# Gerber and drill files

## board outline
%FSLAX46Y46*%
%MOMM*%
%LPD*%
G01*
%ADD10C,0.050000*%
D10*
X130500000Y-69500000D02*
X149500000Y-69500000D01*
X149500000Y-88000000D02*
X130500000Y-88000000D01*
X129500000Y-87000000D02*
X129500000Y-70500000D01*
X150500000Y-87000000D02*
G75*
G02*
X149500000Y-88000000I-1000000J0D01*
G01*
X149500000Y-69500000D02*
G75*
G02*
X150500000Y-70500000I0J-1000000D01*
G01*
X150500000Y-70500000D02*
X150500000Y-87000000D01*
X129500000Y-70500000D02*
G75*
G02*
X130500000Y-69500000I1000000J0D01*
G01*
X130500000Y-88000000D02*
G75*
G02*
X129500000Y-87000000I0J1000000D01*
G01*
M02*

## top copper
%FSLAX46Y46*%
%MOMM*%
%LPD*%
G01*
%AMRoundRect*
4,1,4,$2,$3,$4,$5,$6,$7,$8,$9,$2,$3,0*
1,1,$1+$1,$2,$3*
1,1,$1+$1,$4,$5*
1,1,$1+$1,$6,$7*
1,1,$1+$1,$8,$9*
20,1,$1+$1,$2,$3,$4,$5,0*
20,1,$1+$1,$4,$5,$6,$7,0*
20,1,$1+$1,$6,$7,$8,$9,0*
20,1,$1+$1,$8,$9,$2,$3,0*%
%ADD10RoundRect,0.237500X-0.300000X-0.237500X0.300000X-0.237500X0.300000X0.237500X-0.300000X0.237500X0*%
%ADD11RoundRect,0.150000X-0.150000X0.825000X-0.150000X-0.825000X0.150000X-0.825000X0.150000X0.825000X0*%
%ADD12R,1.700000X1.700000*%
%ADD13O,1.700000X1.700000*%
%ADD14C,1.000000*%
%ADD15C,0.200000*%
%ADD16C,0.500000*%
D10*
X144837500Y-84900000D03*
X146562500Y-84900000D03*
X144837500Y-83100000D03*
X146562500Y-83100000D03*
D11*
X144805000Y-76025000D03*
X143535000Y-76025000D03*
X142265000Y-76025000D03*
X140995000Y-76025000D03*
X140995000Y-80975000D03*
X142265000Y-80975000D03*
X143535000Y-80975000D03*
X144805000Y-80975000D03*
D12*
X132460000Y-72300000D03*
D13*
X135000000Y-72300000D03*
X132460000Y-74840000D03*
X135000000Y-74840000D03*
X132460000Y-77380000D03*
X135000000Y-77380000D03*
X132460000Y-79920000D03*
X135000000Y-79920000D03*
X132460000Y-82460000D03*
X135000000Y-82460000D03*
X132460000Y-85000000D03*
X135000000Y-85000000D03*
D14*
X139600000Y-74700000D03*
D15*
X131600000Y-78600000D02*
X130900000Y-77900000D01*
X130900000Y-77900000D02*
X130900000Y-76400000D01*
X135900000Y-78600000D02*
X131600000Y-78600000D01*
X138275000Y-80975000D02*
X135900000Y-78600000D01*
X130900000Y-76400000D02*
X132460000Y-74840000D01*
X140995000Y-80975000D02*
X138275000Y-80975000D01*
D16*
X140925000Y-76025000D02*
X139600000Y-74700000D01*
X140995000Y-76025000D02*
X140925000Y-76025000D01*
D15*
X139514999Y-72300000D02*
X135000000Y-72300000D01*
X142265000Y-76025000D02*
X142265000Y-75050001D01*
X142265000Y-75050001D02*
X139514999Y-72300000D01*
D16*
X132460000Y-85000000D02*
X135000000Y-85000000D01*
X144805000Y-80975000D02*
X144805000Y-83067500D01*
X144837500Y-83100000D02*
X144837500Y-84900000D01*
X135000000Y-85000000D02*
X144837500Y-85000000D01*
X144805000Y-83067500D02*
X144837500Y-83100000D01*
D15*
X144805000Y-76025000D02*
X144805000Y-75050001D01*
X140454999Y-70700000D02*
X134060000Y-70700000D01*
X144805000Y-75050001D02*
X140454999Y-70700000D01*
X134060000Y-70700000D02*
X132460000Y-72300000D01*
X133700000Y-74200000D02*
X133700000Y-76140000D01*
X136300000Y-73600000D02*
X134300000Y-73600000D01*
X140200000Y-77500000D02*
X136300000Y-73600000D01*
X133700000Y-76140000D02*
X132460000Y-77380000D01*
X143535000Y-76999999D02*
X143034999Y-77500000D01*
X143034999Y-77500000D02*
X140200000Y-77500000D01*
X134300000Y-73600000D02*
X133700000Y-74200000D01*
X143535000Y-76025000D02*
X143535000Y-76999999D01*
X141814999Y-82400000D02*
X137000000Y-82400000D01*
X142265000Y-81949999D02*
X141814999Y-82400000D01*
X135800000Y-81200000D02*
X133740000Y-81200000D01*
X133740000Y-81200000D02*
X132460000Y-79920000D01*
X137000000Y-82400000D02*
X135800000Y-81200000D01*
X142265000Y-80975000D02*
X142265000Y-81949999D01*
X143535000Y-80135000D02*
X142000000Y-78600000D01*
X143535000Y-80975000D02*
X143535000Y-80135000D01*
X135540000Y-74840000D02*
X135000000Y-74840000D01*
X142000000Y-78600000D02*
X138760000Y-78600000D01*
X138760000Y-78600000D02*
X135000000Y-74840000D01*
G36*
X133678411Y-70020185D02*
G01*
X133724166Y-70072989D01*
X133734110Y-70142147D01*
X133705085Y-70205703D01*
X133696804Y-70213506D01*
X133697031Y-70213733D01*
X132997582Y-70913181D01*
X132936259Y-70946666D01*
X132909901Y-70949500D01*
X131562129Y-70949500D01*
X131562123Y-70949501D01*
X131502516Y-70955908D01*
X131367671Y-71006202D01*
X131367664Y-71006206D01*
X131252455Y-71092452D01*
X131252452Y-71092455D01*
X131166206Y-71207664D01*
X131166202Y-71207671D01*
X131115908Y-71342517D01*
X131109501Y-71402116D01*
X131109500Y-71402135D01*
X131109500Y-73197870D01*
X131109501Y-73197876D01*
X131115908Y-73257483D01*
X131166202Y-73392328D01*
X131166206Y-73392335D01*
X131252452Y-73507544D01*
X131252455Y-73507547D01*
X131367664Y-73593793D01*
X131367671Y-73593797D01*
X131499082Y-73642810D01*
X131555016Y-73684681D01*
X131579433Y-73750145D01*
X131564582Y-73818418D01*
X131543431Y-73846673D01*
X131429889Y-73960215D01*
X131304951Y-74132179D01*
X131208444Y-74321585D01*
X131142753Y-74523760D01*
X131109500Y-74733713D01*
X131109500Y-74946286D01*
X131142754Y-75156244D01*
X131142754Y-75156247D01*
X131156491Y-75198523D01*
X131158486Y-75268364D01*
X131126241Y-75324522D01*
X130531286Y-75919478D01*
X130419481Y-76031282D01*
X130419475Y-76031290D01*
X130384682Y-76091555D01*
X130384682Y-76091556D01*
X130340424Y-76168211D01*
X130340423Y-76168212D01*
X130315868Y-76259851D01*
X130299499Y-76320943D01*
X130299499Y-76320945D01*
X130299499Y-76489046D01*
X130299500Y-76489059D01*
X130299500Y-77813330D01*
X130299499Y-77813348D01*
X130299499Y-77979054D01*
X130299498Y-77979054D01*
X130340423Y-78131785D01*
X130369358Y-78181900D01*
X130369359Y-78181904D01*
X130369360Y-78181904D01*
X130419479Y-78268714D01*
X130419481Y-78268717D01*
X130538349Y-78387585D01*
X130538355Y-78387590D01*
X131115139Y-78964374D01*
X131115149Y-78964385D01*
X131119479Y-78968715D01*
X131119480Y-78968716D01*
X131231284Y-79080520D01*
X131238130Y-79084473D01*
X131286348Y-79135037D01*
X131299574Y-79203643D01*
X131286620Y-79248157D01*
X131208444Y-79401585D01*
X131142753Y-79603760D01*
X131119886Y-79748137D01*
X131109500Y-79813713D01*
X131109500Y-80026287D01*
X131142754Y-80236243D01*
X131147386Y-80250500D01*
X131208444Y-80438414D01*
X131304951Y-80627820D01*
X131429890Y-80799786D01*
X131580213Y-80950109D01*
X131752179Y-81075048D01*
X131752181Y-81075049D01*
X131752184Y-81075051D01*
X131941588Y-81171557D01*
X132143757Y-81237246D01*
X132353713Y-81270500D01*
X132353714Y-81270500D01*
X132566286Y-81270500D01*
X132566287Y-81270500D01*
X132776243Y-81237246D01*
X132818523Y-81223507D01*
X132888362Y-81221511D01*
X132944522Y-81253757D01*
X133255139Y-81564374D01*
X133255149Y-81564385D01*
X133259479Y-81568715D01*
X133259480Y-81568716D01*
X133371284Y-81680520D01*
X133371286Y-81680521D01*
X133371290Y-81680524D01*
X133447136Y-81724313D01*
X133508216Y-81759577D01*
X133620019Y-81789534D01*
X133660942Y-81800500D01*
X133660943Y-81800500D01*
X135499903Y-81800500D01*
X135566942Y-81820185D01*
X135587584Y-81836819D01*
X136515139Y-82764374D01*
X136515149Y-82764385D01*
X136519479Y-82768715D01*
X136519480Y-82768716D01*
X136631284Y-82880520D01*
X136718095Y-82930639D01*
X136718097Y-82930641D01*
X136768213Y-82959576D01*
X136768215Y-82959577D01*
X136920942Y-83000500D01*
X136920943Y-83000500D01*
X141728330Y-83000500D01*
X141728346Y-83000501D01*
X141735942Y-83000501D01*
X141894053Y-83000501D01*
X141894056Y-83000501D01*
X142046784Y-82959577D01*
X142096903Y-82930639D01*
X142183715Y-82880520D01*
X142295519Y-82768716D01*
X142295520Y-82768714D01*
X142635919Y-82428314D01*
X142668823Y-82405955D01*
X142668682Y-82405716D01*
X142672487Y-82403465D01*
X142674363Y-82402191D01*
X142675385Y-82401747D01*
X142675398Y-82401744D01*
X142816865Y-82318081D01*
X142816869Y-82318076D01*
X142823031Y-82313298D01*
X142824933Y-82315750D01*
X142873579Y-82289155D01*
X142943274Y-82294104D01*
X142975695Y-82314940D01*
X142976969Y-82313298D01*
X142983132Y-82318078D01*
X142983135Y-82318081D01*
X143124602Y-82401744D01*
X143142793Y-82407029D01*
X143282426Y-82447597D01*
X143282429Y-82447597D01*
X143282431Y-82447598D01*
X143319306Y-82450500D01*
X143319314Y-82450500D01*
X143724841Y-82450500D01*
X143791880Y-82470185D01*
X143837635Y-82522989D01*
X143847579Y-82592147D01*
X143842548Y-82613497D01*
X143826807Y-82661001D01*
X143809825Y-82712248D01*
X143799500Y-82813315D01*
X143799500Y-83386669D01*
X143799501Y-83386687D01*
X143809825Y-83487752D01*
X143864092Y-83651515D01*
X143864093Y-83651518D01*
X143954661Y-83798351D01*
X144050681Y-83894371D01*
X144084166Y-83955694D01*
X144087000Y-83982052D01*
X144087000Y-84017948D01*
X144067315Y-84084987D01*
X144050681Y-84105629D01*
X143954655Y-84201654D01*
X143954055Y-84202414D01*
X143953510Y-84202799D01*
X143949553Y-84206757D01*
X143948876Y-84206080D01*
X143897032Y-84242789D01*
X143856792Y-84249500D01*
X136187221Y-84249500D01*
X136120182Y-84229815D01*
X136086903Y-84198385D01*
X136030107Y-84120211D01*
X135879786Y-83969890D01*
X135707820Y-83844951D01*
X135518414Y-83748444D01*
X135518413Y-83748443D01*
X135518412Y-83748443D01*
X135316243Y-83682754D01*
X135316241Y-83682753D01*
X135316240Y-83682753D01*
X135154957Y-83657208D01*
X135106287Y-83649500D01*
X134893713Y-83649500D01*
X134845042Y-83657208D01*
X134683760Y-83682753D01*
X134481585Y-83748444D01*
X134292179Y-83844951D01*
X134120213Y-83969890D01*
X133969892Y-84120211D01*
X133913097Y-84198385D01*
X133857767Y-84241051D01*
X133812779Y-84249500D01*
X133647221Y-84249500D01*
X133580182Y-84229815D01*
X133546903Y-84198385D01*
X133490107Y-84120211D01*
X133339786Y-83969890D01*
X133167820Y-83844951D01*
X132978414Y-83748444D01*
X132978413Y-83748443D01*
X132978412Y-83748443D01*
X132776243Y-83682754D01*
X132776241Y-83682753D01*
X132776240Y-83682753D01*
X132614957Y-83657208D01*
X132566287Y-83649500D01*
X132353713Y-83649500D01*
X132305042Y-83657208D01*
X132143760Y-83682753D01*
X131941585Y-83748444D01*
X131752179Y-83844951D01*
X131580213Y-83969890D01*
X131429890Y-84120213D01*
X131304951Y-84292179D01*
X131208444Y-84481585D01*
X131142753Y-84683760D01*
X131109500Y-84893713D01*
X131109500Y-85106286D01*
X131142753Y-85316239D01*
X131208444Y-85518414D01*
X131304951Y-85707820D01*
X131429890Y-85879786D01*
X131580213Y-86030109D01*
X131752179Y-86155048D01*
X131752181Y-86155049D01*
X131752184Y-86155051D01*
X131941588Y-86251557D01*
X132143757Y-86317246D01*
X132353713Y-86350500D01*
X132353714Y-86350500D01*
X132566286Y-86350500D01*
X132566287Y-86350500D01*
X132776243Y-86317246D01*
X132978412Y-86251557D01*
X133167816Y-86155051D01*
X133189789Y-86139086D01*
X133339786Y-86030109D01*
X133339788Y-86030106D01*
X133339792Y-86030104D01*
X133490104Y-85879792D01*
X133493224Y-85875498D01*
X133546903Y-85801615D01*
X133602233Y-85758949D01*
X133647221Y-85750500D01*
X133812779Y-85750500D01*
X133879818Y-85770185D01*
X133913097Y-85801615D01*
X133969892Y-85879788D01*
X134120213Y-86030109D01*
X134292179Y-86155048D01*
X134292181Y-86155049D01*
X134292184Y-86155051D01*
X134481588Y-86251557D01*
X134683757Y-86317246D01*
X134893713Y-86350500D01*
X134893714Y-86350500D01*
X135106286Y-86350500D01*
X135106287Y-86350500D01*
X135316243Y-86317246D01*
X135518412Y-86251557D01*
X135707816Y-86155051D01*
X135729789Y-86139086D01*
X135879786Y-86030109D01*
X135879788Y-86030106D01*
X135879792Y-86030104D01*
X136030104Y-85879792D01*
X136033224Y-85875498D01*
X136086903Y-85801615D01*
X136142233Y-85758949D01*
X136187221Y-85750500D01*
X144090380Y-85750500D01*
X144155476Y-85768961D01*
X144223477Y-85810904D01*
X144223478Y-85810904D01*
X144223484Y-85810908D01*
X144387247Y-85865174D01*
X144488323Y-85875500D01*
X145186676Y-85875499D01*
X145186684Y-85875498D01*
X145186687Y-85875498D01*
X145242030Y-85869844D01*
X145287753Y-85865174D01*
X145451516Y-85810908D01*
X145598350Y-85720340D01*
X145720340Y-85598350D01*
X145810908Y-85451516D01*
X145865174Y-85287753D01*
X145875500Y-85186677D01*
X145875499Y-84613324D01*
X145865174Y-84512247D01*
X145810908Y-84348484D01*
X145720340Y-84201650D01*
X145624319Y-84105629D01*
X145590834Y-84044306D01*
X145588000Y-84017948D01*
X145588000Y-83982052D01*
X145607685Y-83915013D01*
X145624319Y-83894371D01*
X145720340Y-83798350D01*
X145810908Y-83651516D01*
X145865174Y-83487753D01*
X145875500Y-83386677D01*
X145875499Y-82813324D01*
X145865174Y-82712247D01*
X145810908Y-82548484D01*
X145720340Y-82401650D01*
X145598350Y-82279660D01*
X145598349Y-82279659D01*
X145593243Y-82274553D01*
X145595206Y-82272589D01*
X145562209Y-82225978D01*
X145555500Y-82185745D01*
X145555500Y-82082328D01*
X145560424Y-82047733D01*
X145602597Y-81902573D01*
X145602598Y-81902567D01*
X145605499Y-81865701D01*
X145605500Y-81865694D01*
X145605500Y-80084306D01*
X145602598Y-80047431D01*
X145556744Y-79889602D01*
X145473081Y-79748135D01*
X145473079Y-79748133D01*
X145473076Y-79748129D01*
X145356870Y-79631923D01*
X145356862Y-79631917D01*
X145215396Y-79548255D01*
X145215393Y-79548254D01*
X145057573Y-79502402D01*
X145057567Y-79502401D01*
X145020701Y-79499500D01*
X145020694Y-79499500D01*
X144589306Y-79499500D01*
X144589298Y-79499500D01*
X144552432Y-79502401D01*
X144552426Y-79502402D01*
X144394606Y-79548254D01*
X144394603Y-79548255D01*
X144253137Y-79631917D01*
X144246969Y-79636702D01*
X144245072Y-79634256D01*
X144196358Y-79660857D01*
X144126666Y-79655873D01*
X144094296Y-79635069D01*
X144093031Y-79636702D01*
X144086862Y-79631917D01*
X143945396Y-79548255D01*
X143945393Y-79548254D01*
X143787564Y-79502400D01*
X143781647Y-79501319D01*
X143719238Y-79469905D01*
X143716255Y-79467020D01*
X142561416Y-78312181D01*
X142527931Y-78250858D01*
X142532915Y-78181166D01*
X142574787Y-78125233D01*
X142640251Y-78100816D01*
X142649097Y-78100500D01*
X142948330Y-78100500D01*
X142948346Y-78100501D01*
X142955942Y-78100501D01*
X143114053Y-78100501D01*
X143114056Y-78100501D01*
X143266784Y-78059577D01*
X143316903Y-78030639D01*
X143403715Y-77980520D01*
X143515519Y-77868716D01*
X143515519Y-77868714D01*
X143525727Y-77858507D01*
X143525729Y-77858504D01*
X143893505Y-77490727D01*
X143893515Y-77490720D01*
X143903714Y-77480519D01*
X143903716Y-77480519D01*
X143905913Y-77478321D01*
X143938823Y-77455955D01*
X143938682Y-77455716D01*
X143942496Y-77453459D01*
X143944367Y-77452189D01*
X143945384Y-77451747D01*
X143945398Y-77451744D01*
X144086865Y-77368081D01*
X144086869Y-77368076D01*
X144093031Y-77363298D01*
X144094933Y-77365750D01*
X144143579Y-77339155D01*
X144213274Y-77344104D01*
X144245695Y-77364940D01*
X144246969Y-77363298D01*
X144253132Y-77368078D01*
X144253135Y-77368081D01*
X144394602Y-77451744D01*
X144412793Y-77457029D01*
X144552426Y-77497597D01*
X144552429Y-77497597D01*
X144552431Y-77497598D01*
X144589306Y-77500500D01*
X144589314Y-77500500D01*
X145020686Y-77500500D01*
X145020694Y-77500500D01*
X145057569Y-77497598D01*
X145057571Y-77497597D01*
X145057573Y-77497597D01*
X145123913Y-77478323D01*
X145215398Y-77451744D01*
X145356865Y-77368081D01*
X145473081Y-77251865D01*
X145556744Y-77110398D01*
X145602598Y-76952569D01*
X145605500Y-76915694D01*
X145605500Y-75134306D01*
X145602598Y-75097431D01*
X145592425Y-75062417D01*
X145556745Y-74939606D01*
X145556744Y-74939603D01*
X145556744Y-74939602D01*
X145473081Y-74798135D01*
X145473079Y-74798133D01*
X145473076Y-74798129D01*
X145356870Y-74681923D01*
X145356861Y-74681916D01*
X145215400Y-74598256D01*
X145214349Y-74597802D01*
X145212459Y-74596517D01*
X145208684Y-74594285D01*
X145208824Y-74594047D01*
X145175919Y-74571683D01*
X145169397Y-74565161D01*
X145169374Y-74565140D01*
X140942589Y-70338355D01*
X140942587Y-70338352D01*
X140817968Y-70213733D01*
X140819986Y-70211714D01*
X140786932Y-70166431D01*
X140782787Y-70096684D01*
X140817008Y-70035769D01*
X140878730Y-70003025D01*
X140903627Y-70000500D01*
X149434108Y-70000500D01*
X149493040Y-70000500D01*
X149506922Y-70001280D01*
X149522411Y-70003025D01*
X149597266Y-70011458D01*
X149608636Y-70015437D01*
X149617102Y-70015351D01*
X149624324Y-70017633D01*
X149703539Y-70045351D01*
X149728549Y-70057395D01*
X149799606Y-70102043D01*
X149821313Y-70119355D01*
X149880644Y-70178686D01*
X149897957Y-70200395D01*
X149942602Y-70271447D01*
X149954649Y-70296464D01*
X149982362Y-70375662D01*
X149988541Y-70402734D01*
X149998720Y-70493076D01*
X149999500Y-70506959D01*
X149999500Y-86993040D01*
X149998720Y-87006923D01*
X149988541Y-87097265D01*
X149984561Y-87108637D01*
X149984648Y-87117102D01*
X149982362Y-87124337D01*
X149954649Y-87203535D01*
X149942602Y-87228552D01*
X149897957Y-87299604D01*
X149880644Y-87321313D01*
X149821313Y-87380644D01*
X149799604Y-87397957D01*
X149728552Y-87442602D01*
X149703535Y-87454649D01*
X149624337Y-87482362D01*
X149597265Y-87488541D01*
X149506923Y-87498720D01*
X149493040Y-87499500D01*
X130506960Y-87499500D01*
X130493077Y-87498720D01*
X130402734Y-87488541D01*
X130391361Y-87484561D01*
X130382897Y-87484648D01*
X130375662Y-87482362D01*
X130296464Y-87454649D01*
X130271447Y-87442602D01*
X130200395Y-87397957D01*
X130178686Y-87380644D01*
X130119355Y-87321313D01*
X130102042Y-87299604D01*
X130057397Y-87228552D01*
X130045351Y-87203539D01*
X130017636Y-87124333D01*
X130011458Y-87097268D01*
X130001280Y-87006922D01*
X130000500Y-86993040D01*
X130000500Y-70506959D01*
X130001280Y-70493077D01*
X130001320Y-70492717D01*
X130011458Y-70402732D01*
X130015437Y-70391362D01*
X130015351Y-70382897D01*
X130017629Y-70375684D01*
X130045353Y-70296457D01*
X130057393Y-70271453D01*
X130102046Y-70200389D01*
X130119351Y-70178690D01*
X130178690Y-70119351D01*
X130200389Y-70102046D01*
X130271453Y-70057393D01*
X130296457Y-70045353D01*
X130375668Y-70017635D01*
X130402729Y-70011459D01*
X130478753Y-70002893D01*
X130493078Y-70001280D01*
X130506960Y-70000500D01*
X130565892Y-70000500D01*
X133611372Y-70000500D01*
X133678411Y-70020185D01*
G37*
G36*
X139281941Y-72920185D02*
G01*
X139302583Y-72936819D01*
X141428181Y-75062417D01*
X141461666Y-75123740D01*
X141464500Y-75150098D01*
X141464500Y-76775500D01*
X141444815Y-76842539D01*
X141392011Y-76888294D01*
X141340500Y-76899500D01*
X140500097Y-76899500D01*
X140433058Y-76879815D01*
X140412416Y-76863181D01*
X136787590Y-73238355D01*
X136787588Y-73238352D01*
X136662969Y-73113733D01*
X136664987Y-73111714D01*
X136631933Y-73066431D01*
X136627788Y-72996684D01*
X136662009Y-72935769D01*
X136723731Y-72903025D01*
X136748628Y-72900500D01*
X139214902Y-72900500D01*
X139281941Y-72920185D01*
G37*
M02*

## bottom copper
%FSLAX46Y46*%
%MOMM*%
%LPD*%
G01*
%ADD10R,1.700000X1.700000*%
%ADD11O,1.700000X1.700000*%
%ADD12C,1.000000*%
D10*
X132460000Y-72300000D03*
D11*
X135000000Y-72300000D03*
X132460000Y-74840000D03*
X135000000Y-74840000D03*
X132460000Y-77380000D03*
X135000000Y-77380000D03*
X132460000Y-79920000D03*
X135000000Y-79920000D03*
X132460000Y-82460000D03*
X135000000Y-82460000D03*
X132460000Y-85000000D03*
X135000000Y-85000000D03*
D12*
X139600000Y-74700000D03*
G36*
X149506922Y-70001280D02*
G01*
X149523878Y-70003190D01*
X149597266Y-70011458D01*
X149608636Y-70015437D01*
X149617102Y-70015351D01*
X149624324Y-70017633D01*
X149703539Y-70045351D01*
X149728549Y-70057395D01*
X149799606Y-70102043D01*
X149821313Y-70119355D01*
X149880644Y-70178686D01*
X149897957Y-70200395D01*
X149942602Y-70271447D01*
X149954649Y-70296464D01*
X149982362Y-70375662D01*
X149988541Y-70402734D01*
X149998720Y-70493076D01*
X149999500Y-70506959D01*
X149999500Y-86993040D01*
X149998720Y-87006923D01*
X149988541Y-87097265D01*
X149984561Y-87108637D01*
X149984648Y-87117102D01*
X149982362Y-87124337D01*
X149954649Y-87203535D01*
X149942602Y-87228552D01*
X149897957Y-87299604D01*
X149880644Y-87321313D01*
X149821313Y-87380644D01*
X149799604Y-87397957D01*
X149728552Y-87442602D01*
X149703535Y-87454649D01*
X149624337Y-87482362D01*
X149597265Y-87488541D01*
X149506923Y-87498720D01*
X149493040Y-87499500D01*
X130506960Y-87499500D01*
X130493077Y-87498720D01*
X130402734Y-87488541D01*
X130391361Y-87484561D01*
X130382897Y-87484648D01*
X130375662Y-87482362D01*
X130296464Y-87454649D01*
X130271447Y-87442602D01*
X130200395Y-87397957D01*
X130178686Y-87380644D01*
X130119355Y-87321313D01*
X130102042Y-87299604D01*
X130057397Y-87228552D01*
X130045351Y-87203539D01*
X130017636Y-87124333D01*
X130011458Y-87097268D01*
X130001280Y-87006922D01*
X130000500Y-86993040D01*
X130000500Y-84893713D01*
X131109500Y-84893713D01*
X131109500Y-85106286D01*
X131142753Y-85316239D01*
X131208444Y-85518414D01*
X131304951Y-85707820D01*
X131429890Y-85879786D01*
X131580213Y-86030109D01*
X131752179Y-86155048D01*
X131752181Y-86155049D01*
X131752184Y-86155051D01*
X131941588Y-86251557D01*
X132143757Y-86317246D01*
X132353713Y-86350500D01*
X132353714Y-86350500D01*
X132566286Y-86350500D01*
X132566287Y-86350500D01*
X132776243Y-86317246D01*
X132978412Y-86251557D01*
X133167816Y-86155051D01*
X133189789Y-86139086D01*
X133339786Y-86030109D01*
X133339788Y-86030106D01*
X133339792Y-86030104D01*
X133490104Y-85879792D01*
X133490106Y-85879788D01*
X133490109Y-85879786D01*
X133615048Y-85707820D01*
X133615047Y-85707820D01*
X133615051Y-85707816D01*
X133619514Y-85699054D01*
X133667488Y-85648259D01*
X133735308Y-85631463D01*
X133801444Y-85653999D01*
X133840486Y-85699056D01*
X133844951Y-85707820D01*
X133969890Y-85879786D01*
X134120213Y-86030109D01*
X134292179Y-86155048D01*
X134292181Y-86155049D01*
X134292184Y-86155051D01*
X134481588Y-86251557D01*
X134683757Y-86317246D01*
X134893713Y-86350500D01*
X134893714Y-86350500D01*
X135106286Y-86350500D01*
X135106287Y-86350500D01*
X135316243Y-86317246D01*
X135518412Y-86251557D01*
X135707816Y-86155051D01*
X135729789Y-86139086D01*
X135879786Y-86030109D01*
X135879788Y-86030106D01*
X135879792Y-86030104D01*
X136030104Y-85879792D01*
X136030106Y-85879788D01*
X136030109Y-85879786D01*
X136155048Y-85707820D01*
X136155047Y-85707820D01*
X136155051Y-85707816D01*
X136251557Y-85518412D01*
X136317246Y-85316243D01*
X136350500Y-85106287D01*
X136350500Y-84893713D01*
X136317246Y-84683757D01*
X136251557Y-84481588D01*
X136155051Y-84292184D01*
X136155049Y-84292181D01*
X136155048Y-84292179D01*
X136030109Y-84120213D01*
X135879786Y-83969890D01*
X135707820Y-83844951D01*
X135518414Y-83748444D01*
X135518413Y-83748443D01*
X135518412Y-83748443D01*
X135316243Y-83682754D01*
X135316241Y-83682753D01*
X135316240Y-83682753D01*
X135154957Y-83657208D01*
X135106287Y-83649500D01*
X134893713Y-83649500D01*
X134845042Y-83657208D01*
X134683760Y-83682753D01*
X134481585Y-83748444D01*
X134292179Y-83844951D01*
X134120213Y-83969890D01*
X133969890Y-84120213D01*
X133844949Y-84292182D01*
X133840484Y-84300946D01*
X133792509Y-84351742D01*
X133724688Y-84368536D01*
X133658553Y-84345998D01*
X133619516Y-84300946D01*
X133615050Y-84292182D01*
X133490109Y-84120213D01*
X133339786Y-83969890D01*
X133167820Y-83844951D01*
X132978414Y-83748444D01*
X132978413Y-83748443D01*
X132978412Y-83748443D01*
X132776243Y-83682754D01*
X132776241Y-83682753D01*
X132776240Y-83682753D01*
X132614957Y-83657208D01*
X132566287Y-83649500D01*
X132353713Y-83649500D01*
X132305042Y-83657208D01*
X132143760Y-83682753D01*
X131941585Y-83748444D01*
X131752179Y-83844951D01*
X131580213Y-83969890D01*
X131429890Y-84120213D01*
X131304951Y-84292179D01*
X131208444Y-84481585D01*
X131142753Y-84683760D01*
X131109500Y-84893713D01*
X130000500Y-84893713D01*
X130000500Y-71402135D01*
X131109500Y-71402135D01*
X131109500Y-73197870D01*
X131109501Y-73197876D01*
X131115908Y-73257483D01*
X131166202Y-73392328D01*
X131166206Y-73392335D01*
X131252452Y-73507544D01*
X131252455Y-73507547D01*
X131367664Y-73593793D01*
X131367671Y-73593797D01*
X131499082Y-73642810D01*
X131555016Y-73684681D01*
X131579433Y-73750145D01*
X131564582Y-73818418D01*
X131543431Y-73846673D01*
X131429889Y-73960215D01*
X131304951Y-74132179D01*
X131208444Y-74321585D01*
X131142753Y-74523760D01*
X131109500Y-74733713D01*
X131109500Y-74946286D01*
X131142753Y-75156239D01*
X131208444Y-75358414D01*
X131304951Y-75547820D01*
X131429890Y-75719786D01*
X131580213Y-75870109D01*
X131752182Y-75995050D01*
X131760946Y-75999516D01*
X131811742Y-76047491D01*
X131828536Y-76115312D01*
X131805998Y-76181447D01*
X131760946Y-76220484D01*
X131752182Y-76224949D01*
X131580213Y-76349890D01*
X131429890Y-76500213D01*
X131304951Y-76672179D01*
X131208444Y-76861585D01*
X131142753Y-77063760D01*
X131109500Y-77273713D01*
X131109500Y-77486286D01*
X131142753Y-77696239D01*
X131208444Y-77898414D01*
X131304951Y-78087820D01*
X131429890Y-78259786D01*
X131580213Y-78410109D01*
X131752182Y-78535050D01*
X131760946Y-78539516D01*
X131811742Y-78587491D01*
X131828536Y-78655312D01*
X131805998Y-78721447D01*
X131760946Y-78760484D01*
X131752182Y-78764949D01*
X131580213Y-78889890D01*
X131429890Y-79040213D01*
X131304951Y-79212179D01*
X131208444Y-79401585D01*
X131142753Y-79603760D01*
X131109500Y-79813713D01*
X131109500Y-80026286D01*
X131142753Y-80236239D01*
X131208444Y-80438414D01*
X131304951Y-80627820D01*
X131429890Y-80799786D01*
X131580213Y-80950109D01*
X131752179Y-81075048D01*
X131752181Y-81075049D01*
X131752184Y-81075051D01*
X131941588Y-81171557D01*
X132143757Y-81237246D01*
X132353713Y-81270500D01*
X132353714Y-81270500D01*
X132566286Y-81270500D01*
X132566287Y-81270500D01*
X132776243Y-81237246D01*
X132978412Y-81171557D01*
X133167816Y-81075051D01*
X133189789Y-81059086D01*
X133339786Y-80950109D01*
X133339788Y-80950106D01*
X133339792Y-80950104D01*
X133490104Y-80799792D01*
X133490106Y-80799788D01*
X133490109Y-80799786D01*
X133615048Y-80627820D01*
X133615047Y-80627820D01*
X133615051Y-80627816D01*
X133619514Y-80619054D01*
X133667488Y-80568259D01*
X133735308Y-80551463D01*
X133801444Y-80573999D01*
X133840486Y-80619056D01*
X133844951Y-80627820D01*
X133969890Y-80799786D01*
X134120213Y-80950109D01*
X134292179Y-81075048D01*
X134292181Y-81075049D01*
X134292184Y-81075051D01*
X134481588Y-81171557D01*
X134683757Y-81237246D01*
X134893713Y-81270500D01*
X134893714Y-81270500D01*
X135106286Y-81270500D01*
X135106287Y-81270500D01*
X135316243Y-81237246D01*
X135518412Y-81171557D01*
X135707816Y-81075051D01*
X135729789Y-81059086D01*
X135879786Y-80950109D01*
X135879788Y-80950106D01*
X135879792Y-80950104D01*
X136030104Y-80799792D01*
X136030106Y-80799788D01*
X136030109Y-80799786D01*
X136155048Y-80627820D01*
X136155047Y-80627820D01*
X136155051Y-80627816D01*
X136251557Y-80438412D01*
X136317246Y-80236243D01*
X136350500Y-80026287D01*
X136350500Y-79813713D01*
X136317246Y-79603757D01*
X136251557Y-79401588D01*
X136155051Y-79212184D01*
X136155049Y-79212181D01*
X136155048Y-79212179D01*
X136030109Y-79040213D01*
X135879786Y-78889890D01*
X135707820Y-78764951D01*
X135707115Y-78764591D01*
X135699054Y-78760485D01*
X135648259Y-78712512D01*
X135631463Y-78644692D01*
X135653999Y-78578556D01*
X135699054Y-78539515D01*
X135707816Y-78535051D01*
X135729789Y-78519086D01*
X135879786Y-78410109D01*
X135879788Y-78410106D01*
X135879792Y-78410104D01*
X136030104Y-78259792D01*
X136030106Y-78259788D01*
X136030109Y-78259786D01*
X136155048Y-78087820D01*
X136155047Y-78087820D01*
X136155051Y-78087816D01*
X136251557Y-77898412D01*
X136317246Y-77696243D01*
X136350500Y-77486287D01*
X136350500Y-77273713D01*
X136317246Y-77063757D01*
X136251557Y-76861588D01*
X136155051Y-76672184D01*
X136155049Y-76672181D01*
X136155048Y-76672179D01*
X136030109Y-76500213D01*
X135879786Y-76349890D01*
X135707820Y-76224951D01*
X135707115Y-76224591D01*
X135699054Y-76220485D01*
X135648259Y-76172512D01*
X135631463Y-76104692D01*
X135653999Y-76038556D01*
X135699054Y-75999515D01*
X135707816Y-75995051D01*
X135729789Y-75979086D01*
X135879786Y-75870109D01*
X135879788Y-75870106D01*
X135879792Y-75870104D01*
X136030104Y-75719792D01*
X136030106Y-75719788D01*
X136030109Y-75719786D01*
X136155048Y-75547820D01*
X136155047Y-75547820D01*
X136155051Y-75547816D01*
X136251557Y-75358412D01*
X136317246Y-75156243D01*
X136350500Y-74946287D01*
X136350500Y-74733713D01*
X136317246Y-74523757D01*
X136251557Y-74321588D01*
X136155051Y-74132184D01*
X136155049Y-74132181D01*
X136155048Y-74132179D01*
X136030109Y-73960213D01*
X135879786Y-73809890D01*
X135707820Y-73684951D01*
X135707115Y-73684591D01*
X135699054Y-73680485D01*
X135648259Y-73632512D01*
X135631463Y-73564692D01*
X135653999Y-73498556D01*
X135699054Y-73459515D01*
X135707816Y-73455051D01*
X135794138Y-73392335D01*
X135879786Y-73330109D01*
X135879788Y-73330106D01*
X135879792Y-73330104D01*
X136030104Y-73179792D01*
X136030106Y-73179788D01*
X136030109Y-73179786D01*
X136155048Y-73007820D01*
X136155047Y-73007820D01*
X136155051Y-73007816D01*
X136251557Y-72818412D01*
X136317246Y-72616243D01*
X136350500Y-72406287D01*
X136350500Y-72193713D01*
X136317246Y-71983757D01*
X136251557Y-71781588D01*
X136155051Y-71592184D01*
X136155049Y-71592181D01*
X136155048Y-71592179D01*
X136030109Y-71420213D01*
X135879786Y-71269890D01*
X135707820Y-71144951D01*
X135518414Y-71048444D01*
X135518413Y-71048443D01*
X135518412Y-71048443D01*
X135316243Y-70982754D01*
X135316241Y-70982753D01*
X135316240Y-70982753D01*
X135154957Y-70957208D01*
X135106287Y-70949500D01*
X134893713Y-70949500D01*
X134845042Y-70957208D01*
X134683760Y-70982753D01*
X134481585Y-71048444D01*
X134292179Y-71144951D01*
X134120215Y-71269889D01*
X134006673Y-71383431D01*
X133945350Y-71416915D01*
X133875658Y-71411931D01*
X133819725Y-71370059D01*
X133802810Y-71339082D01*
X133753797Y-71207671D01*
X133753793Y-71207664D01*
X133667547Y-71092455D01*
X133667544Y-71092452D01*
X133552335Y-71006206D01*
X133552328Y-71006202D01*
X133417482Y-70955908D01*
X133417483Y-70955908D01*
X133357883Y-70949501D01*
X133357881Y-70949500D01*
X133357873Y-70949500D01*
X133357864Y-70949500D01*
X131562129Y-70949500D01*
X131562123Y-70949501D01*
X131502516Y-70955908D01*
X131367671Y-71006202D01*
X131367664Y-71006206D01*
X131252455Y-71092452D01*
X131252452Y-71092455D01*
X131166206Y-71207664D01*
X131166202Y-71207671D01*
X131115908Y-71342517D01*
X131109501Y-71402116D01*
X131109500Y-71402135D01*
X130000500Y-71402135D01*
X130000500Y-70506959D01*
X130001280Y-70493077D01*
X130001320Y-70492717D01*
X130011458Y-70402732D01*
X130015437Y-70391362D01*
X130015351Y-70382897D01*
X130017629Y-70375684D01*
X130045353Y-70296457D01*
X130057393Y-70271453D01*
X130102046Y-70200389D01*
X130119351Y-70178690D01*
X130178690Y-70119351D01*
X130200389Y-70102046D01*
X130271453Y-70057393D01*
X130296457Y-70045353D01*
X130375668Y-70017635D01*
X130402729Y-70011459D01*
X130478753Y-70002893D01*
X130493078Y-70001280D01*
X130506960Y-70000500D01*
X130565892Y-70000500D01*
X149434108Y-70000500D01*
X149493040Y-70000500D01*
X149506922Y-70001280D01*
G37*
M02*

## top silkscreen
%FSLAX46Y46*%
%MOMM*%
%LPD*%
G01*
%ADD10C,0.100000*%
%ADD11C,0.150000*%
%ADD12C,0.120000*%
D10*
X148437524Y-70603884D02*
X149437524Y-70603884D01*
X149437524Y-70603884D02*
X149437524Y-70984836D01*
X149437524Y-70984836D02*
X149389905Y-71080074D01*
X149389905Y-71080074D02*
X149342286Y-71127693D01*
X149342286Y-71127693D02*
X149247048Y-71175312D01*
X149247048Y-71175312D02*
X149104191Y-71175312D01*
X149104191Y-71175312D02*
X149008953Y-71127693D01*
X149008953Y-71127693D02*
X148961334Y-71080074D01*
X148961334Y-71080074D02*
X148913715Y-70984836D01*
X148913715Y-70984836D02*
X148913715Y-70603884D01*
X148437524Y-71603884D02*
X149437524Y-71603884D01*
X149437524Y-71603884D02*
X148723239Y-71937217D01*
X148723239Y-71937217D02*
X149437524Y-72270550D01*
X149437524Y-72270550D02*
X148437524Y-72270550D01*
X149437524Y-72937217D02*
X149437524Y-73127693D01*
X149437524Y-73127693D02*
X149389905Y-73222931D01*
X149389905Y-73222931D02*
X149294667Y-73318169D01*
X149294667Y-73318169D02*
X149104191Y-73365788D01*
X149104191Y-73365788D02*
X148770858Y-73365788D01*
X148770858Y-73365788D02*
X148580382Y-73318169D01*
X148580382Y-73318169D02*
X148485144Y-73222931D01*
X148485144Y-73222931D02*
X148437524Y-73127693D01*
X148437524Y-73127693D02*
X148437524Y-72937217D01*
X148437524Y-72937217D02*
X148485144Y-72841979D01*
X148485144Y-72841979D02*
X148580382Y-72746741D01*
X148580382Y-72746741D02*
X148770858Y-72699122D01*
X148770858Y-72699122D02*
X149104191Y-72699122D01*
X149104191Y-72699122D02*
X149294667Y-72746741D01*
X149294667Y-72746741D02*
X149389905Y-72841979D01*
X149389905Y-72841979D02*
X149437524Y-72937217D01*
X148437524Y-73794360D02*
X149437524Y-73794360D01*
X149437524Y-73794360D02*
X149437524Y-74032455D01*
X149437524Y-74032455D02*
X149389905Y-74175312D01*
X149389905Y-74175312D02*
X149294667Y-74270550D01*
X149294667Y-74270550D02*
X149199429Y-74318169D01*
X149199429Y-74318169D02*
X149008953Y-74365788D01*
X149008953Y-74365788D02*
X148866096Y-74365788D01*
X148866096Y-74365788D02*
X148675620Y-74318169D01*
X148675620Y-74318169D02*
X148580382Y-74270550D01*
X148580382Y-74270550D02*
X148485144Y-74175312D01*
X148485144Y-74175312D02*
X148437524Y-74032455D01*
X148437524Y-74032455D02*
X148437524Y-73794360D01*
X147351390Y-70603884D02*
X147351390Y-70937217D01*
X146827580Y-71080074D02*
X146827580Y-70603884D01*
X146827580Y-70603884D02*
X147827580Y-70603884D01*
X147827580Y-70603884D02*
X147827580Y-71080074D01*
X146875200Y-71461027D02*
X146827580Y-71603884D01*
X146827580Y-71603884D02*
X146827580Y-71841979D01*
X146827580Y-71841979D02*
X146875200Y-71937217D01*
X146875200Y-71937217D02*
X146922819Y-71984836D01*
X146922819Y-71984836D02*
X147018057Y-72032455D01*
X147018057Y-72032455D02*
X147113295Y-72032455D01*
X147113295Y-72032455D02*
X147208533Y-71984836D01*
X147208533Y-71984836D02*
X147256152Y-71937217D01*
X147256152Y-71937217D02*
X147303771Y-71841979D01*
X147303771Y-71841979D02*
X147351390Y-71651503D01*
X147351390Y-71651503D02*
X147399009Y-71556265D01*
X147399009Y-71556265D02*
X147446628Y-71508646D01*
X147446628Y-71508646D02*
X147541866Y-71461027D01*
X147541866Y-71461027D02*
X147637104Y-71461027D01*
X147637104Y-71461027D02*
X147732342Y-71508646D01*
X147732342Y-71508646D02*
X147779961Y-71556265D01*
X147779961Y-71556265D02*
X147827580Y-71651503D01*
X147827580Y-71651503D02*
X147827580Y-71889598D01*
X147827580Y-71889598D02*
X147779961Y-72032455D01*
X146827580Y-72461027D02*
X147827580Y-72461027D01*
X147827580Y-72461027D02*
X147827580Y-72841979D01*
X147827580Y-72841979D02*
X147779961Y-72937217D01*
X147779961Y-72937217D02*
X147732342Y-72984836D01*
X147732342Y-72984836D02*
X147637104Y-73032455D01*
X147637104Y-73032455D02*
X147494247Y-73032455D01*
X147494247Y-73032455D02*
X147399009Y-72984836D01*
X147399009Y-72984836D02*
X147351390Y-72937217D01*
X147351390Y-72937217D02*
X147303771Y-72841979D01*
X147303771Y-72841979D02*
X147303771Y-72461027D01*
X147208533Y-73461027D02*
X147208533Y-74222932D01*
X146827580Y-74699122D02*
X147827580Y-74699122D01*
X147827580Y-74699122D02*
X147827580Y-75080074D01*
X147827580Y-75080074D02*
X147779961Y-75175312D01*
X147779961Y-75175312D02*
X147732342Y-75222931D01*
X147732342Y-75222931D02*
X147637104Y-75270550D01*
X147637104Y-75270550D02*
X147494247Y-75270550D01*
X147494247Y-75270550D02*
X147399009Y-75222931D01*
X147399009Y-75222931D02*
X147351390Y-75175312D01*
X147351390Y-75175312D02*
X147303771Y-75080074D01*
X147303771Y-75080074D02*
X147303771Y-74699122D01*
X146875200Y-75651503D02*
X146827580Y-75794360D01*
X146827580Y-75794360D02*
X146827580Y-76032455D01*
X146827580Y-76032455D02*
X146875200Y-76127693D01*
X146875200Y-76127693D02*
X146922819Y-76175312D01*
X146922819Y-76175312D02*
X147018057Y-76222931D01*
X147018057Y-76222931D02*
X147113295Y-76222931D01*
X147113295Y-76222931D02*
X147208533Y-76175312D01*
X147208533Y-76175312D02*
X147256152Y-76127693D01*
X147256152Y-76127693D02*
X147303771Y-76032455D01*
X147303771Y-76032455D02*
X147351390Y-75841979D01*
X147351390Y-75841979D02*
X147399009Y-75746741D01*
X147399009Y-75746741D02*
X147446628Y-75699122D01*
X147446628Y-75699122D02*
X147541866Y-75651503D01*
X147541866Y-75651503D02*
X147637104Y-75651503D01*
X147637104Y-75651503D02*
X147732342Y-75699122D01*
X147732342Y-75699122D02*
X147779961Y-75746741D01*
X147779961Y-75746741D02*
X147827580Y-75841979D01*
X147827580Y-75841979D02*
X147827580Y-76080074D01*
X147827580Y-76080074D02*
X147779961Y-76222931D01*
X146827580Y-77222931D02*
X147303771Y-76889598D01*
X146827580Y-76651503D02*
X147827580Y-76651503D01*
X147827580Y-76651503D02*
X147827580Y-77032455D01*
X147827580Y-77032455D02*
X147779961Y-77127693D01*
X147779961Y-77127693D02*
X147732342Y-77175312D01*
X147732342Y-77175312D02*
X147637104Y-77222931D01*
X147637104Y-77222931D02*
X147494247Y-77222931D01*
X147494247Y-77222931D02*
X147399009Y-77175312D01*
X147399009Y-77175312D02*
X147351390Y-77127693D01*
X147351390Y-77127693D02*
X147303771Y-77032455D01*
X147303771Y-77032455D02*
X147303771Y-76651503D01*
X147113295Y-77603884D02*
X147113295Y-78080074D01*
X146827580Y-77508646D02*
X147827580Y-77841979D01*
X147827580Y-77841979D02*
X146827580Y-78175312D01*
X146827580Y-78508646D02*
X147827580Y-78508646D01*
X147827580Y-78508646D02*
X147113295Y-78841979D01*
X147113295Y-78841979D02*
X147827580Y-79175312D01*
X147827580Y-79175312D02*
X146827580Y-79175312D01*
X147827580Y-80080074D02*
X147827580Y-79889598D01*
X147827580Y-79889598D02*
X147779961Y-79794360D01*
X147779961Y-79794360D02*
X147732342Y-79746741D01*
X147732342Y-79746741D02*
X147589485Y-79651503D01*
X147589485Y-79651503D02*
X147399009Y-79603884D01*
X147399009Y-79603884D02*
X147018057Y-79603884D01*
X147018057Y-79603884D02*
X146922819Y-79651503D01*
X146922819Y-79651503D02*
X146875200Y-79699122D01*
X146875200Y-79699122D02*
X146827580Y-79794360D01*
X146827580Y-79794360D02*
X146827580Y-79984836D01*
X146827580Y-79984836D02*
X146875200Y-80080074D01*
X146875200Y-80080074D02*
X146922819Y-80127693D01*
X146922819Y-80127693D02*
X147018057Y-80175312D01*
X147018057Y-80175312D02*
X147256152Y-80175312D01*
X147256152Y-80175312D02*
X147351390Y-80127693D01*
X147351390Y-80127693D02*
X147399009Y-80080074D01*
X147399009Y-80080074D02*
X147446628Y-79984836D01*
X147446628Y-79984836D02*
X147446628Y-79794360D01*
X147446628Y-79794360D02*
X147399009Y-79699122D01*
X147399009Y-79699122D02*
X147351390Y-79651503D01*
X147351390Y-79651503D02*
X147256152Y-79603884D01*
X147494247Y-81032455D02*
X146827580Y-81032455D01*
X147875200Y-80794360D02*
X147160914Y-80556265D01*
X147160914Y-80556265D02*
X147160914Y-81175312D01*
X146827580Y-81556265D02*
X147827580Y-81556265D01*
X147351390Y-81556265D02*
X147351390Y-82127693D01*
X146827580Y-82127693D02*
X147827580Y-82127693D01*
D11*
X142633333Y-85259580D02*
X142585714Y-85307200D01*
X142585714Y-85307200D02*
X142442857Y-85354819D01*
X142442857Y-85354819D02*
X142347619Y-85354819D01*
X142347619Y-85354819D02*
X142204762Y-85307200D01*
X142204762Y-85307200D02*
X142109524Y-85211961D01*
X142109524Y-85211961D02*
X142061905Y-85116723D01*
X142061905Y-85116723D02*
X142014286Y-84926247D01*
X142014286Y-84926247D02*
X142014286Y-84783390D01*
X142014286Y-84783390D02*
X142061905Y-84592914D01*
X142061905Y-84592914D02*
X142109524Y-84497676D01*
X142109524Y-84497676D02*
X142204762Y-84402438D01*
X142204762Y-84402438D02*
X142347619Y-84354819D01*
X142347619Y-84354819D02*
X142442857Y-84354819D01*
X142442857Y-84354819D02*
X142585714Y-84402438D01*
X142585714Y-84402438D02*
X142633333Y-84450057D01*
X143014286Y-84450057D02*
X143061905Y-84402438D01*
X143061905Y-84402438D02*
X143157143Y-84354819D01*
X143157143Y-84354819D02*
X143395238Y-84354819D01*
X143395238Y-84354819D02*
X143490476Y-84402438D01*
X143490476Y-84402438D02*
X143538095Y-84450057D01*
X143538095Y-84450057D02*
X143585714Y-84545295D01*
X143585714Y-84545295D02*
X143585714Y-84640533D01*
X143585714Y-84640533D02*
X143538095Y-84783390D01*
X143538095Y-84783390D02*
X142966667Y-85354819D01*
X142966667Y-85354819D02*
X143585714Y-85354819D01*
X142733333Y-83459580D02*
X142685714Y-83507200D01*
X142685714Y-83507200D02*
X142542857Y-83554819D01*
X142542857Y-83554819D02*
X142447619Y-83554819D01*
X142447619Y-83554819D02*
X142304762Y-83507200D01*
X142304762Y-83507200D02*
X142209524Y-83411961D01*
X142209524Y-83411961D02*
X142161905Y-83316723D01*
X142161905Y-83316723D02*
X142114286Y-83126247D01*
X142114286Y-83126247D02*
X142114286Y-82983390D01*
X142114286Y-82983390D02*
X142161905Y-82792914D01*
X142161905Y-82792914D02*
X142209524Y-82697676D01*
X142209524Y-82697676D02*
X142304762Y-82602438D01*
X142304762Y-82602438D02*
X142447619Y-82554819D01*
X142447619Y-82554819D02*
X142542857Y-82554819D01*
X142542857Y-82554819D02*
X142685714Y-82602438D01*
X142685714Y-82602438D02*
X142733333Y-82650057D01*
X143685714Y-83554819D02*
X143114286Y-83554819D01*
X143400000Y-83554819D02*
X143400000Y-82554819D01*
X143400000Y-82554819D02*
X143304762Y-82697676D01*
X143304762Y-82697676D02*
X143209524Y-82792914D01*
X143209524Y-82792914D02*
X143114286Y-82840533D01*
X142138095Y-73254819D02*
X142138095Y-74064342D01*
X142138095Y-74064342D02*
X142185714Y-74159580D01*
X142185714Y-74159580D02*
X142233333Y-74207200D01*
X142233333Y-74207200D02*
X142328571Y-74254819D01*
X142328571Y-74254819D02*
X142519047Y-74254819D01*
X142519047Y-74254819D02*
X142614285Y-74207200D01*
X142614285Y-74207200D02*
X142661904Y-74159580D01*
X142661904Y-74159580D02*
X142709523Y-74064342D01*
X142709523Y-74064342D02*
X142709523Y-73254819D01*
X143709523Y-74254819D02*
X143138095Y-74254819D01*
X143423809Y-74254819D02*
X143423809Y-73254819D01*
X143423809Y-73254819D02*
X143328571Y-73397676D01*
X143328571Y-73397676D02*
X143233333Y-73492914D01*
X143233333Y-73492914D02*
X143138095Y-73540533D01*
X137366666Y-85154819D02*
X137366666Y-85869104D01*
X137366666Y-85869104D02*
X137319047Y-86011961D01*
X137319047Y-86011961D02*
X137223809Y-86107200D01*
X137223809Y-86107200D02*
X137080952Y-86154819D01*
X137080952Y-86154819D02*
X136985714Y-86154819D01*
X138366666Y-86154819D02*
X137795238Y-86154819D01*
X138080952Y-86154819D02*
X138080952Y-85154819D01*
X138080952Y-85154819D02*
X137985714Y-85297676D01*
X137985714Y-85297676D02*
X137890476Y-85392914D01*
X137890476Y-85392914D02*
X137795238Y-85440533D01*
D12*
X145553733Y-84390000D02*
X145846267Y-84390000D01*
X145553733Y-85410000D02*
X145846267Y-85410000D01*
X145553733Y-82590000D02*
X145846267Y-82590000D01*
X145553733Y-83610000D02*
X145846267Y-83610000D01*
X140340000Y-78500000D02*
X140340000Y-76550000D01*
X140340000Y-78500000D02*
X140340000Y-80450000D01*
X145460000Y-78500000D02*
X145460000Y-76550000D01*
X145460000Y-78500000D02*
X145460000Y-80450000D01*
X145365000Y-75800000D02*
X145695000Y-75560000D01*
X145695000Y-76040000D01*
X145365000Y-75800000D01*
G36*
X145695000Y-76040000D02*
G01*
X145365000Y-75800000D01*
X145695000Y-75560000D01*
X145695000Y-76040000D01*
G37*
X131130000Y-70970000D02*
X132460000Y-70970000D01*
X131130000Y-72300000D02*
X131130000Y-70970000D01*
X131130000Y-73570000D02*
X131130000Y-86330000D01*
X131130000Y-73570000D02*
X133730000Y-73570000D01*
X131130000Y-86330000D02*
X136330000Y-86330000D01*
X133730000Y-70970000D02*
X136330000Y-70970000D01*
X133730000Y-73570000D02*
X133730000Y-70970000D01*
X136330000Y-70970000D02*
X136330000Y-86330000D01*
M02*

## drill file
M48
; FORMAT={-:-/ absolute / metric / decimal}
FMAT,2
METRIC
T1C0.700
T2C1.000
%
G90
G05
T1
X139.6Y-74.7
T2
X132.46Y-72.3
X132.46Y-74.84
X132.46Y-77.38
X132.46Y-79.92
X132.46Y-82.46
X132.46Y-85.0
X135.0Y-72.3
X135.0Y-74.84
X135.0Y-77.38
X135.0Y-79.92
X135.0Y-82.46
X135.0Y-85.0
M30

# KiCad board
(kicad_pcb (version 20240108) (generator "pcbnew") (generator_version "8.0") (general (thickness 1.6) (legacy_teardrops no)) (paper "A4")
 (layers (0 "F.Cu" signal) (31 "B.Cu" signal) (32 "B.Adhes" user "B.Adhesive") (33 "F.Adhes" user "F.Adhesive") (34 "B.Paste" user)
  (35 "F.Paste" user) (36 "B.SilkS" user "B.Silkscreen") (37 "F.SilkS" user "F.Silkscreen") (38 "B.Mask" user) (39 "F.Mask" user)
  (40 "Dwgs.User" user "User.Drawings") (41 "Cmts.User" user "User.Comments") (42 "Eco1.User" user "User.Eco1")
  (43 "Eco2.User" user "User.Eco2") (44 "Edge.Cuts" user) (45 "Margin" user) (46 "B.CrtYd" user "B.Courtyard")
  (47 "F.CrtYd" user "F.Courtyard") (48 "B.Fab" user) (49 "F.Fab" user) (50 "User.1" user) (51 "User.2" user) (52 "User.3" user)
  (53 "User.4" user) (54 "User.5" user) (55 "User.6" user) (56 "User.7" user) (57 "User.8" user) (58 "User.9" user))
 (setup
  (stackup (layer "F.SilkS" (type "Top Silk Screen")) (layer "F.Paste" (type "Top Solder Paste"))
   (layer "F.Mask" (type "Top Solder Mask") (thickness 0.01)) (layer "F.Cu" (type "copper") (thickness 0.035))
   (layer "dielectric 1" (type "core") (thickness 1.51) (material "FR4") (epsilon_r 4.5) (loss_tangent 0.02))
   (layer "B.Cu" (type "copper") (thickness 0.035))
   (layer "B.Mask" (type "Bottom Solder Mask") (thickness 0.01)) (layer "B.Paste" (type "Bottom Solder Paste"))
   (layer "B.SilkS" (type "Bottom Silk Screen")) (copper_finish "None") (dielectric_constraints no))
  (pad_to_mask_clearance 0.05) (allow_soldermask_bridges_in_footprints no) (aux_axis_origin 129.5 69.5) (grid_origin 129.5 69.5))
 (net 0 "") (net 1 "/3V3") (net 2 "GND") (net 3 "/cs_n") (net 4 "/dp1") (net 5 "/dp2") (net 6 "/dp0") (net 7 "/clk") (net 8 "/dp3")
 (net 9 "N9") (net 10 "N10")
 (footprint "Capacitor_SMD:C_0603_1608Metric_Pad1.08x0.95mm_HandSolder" (layer "F.Cu") (at 145.7 84.9)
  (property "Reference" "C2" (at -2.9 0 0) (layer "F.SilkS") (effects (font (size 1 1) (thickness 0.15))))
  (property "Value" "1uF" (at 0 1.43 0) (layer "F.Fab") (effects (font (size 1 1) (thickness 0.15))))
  (fp_line (start -0.146267 -0.51) (end 0.146267 -0.51) (stroke (width 0.12) (type solid)) (layer "F.SilkS"))
  (fp_line (start -0.146267 0.51) (end 0.146267 0.51) (stroke (width 0.12) (type solid)) (layer "F.SilkS"))
  (pad "1" smd roundrect (at -0.8625 0) (size 1.075 0.95) (layers "F.Cu" "F.Paste" "F.Mask") (roundrect_rratio 0.25) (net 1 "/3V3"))
  (pad "2" smd roundrect (at 0.8625 0) (size 1.075 0.95) (layers "F.Cu" "F.Paste" "F.Mask") (roundrect_rratio 0.25) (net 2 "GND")))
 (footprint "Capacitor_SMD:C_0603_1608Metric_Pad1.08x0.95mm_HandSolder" (layer "F.Cu") (at 145.7 83.1)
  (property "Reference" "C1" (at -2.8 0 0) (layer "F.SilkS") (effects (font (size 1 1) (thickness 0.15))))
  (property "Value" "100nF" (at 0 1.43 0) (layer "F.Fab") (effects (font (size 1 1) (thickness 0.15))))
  (fp_line (start -0.146267 -0.51) (end 0.146267 -0.51) (stroke (width 0.12) (type solid)) (layer "F.SilkS"))
  (fp_line (start -0.146267 0.51) (end 0.146267 0.51) (stroke (width 0.12) (type solid)) (layer "F.SilkS"))
  (pad "1" smd roundrect (at -0.8625 0) (size 1.075 0.95) (layers "F.Cu" "F.Paste" "F.Mask") (roundrect_rratio 0.25) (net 1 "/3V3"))
  (pad "2" smd roundrect (at 0.8625 0) (size 1.075 0.95) (layers "F.Cu" "F.Paste" "F.Mask") (roundrect_rratio 0.25) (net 2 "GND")))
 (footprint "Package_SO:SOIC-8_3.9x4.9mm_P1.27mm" (layer "F.Cu") (at 142.9 78.5 -90)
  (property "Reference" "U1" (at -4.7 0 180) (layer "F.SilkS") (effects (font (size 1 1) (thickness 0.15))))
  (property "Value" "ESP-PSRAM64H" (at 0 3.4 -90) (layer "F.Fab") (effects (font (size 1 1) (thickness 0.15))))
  (fp_line (start 0 2.56) (end -1.95 2.56) (stroke (width 0.12) (type solid)) (layer "F.SilkS"))
  (fp_line (start 0 2.56) (end 1.95 2.56) (stroke (width 0.12) (type solid)) (layer "F.SilkS"))
  (fp_line (start 0 -2.56) (end -1.95 -2.56) (stroke (width 0.12) (type solid)) (layer "F.SilkS"))
  (fp_line (start 0 -2.56) (end 1.95 -2.56) (stroke (width 0.12) (type solid)) (layer "F.SilkS"))
  (fp_poly
   (pts (xy -2.7 -2.465) (xy -2.94 -2.795) (xy -2.46 -2.795) (xy -2.7 -2.465)) (stroke (width 0.12) (type solid)) (fill solid)
   (layer "F.SilkS"))
  (pad "1" smd roundrect (at -2.475 -1.905 270) (size 1.95 0.6) (layers "F.Cu" "F.Paste" "F.Mask") (roundrect_rratio 0.25) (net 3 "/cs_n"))
  (pad "2" smd roundrect (at -2.475 -0.635 270) (size 1.95 0.6) (layers "F.Cu" "F.Paste" "F.Mask") (roundrect_rratio 0.25) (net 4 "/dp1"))
  (pad "3" smd roundrect (at -2.475 0.635 270) (size 1.95 0.6) (layers "F.Cu" "F.Paste" "F.Mask") (roundrect_rratio 0.25) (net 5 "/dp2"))
  (pad "4" smd roundrect (at -2.475 1.905 270) (size 1.95 0.6) (layers "F.Cu" "F.Paste" "F.Mask") (roundrect_rratio 0.25) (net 2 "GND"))
  (pad "5" smd roundrect (at 2.475 1.905 270) (size 1.95 0.6) (layers "F.Cu" "F.Paste" "F.Mask") (roundrect_rratio 0.25) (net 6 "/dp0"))
  (pad "6" smd roundrect (at 2.475 0.635 270) (size 1.95 0.6) (layers "F.Cu" "F.Paste" "F.Mask") (roundrect_rratio 0.25) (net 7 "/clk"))
  (pad "7" smd roundrect (at 2.475 -0.635 270) (size 1.95 0.6) (layers "F.Cu" "F.Paste" "F.Mask") (roundrect_rratio 0.25) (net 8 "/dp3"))
  (pad "8" smd roundrect (at 2.475 -1.905 270) (size 1.95 0.6) (layers "F.Cu" "F.Paste" "F.Mask") (roundrect_rratio 0.25) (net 1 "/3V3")))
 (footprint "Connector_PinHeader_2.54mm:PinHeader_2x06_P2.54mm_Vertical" (layer "F.Cu") (at 132.46 72.3)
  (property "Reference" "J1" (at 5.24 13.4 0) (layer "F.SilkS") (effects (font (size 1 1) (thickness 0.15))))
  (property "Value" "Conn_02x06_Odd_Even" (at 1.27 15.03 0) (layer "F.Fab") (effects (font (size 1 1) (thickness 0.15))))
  (fp_line (start -1.33 -1.33) (end 0 -1.33) (stroke (width 0.12) (type solid)) (layer "F.SilkS"))
  (fp_line (start -1.33 0) (end -1.33 -1.33) (stroke (width 0.12) (type solid)) (layer "F.SilkS"))
  (fp_line (start -1.33 1.27) (end -1.33 14.03) (stroke (width 0.12) (type solid)) (layer "F.SilkS"))
  (fp_line (start -1.33 1.27) (end 1.27 1.27) (stroke (width 0.12) (type solid)) (layer "F.SilkS"))
  (fp_line (start -1.33 14.03) (end 3.87 14.03) (stroke (width 0.12) (type solid)) (layer "F.SilkS"))
  (fp_line (start 1.27 -1.33) (end 3.87 -1.33) (stroke (width 0.12) (type solid)) (layer "F.SilkS"))
  (fp_line (start 1.27 1.27) (end 1.27 -1.33) (stroke (width 0.12) (type solid)) (layer "F.SilkS"))
  (fp_line (start 3.87 -1.33) (end 3.87 14.03) (stroke (width 0.12) (type solid)) (layer "F.SilkS"))
  (pad "1" thru_hole rect (at 0 0) (size 1.7 1.7) (drill 1) (layers "*.Cu" "*.Mask") (remove_unused_layers no) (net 3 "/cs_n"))
  (pad "2" thru_hole oval (at 2.54 0) (size 1.7 1.7) (drill 1) (layers "*.Cu" "*.Mask") (remove_unused_layers no) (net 5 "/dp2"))
  (pad "3" thru_hole oval (at 0 2.54) (size 1.7 1.7) (drill 1) (layers "*.Cu" "*.Mask") (remove_unused_layers no) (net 6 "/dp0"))
  (pad "4" thru_hole oval (at 2.54 2.54) (size 1.7 1.7) (drill 1) (layers "*.Cu" "*.Mask") (remove_unused_layers no) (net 8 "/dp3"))
  (pad "5" thru_hole oval (at 0 5.08) (size 1.7 1.7) (drill 1) (layers "*.Cu" "*.Mask") (remove_unused_layers no) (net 4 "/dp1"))
  (pad "6" thru_hole oval (at 2.54 5.08) (size 1.7 1.7) (drill 1) (layers "*.Cu" "*.Mask") (remove_unused_layers no) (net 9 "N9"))
  (pad "7" thru_hole oval (at 0 7.62) (size 1.7 1.7) (drill 1) (layers "*.Cu" "*.Mask") (remove_unused_layers no) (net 7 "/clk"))
  (pad "8" thru_hole oval (at 2.54 7.62) (size 1.7 1.7) (drill 1) (layers "*.Cu" "*.Mask") (remove_unused_layers no) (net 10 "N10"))
  (pad "9" thru_hole oval (at 0 10.16) (size 1.7 1.7) (drill 1) (layers "*.Cu" "*.Mask") (remove_unused_layers no) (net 2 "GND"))
  (pad "10" thru_hole oval (at 2.54 10.16) (size 1.7 1.7) (drill 1) (layers "*.Cu" "*.Mask") (remove_unused_layers no) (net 2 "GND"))
  (pad "11" thru_hole oval (at 0 12.7) (size 1.7 1.7) (drill 1) (layers "*.Cu" "*.Mask") (remove_unused_layers no) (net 1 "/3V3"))
  (pad "12" thru_hole oval (at 2.54 12.7) (size 1.7 1.7) (drill 1) (layers "*.Cu" "*.Mask") (remove_unused_layers no) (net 1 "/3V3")))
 (gr_line (start 130.5 69.5) (end 149.5 69.5) (stroke (width 0.05) (type default)) (layer "Edge.Cuts"))
 (gr_line (start 149.5 88) (end 130.5 88) (stroke (width 0.05) (type default)) (layer "Edge.Cuts"))
 (gr_line (start 129.5 87) (end 129.5 70.5) (stroke (width 0.05) (type default)) (layer "Edge.Cuts"))
 (gr_arc (start 150.5 87) (mid 150.207107 87.707107) (end 149.5 88) (stroke (width 0.05) (type default)) (layer "Edge.Cuts"))
 (gr_arc (start 149.5 69.5) (mid 150.207107 69.792893) (end 150.5 70.5) (stroke (width 0.05) (type default)) (layer "Edge.Cuts"))
 (gr_line (start 150.5 70.5) (end 150.5 87) (stroke (width 0.05) (type default)) (layer "Edge.Cuts"))
 (gr_arc (start 129.5 70.5) (mid 129.792893 69.792893) (end 130.5 69.5) (stroke (width 0.05) (type default)) (layer "Edge.Cuts"))
 (gr_arc (start 130.5 88) (mid 129.792893 87.707107) (end 129.5 87) (stroke (width 0.05) (type default)) (layer "Edge.Cuts"))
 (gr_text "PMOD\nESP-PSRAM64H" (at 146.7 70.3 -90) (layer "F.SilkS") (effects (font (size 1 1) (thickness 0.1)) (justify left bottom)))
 (segment (start 131.6 78.6) (end 130.9 77.9) (width 0.2) (layer "F.Cu") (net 6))
 (segment (start 130.9 77.9) (end 130.9 76.4) (width 0.2) (layer "F.Cu") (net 6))
 (segment (start 135.9 78.6) (end 131.6 78.6) (width 0.2) (layer "F.Cu") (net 6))
 (segment (start 138.275 80.975) (end 135.9 78.6) (width 0.2) (layer "F.Cu") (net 6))
 (segment (start 130.9 76.4) (end 132.46 74.84) (width 0.2) (layer "F.Cu") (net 6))
 (segment (start 140.995 80.975) (end 138.275 80.975) (width 0.2) (layer "F.Cu") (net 6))
 (segment (start 140.925 76.025) (end 139.6 74.7) (width 0.5) (layer "F.Cu") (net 2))
 (segment (start 140.995 76.025) (end 140.925 76.025) (width 0.5) (layer "F.Cu") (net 2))
 (via (at 139.6 74.7) (size 1) (drill 0.7) (layers "F.Cu" "B.Cu") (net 2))
 (segment (start 139.514999 72.3) (end 135 72.3) (width 0.2) (layer "F.Cu") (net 5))
 (segment (start 142.265 76.025) (end 142.265 75.050001) (width 0.2) (layer "F.Cu") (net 5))
 (segment (start 142.265 75.050001) (end 139.514999 72.3) (width 0.2) (layer "F.Cu") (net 5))
 (segment (start 132.46 85) (end 135 85) (width 0.5) (layer "F.Cu") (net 1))
 (segment (start 144.805 80.975) (end 144.805 83.0675) (width 0.5) (layer "F.Cu") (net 1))
 (segment (start 144.8375 83.1) (end 144.8375 84.9) (width 0.5) (layer "F.Cu") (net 1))
 (segment (start 135 85) (end 144.8375 85) (width 0.5) (layer "F.Cu") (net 1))
 (segment (start 144.805 83.0675) (end 144.8375 83.1) (width 0.5) (layer "F.Cu") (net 1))
 (segment (start 144.805 76.025) (end 144.805 75.050001) (width 0.2) (layer "F.Cu") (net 3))
 (segment (start 140.454999 70.7) (end 134.06 70.7) (width 0.2) (layer "F.Cu") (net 3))
 (segment (start 144.805 75.050001) (end 140.454999 70.7) (width 0.2) (layer "F.Cu") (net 3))
 (segment (start 134.06 70.7) (end 132.46 72.3) (width 0.2) (layer "F.Cu") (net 3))
 (segment (start 133.7 74.2) (end 133.7 76.14) (width 0.2) (layer "F.Cu") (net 4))
 (segment (start 136.3 73.6) (end 134.3 73.6) (width 0.2) (layer "F.Cu") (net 4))
 (segment (start 140.2 77.5) (end 136.3 73.6) (width 0.2) (layer "F.Cu") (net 4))
 (segment (start 133.7 76.14) (end 132.46 77.38) (width 0.2) (layer "F.Cu") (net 4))
 (segment (start 143.535 76.999999) (end 143.034999 77.5) (width 0.2) (layer "F.Cu") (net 4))
 (segment (start 143.034999 77.5) (end 140.2 77.5) (width 0.2) (layer "F.Cu") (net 4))
 (segment (start 134.3 73.6) (end 133.7 74.2) (width 0.2) (layer "F.Cu") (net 4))
 (segment (start 143.535 76.025) (end 143.535 76.999999) (width 0.2) (layer "F.Cu") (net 4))
 (segment (start 141.814999 82.4) (end 137 82.4) (width 0.2) (layer "F.Cu") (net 7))
 (segment (start 142.265 81.949999) (end 141.814999 82.4) (width 0.2) (layer "F.Cu") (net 7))
 (segment (start 135.8 81.2) (end 133.74 81.2) (width 0.2) (layer "F.Cu") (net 7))
 (segment (start 133.74 81.2) (end 132.46 79.92) (width 0.2) (layer "F.Cu") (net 7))
 (segment (start 137 82.4) (end 135.8 81.2) (width 0.2) (layer "F.Cu") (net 7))
 (segment (start 142.265 80.975) (end 142.265 81.949999) (width 0.2) (layer "F.Cu") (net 7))
 (segment (start 143.535 80.135) (end 142 78.6) (width 0.2) (layer "F.Cu") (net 8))
 (segment (start 143.535 80.975) (end 143.535 80.135) (width 0.2) (layer "F.Cu") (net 8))
 (segment (start 135.54 74.84) (end 135 74.84) (width 0.2) (layer "F.Cu") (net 8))
 (segment (start 142 78.6) (end 138.76 78.6) (width 0.2) (layer "F.Cu") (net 8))
 (segment (start 138.76 78.6) (end 135 74.84) (width 0.2) (layer "F.Cu") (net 8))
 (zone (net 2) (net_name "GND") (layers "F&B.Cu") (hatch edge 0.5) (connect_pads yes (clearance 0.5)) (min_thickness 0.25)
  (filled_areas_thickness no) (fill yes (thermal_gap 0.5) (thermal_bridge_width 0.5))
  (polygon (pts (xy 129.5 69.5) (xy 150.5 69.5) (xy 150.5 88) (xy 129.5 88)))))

